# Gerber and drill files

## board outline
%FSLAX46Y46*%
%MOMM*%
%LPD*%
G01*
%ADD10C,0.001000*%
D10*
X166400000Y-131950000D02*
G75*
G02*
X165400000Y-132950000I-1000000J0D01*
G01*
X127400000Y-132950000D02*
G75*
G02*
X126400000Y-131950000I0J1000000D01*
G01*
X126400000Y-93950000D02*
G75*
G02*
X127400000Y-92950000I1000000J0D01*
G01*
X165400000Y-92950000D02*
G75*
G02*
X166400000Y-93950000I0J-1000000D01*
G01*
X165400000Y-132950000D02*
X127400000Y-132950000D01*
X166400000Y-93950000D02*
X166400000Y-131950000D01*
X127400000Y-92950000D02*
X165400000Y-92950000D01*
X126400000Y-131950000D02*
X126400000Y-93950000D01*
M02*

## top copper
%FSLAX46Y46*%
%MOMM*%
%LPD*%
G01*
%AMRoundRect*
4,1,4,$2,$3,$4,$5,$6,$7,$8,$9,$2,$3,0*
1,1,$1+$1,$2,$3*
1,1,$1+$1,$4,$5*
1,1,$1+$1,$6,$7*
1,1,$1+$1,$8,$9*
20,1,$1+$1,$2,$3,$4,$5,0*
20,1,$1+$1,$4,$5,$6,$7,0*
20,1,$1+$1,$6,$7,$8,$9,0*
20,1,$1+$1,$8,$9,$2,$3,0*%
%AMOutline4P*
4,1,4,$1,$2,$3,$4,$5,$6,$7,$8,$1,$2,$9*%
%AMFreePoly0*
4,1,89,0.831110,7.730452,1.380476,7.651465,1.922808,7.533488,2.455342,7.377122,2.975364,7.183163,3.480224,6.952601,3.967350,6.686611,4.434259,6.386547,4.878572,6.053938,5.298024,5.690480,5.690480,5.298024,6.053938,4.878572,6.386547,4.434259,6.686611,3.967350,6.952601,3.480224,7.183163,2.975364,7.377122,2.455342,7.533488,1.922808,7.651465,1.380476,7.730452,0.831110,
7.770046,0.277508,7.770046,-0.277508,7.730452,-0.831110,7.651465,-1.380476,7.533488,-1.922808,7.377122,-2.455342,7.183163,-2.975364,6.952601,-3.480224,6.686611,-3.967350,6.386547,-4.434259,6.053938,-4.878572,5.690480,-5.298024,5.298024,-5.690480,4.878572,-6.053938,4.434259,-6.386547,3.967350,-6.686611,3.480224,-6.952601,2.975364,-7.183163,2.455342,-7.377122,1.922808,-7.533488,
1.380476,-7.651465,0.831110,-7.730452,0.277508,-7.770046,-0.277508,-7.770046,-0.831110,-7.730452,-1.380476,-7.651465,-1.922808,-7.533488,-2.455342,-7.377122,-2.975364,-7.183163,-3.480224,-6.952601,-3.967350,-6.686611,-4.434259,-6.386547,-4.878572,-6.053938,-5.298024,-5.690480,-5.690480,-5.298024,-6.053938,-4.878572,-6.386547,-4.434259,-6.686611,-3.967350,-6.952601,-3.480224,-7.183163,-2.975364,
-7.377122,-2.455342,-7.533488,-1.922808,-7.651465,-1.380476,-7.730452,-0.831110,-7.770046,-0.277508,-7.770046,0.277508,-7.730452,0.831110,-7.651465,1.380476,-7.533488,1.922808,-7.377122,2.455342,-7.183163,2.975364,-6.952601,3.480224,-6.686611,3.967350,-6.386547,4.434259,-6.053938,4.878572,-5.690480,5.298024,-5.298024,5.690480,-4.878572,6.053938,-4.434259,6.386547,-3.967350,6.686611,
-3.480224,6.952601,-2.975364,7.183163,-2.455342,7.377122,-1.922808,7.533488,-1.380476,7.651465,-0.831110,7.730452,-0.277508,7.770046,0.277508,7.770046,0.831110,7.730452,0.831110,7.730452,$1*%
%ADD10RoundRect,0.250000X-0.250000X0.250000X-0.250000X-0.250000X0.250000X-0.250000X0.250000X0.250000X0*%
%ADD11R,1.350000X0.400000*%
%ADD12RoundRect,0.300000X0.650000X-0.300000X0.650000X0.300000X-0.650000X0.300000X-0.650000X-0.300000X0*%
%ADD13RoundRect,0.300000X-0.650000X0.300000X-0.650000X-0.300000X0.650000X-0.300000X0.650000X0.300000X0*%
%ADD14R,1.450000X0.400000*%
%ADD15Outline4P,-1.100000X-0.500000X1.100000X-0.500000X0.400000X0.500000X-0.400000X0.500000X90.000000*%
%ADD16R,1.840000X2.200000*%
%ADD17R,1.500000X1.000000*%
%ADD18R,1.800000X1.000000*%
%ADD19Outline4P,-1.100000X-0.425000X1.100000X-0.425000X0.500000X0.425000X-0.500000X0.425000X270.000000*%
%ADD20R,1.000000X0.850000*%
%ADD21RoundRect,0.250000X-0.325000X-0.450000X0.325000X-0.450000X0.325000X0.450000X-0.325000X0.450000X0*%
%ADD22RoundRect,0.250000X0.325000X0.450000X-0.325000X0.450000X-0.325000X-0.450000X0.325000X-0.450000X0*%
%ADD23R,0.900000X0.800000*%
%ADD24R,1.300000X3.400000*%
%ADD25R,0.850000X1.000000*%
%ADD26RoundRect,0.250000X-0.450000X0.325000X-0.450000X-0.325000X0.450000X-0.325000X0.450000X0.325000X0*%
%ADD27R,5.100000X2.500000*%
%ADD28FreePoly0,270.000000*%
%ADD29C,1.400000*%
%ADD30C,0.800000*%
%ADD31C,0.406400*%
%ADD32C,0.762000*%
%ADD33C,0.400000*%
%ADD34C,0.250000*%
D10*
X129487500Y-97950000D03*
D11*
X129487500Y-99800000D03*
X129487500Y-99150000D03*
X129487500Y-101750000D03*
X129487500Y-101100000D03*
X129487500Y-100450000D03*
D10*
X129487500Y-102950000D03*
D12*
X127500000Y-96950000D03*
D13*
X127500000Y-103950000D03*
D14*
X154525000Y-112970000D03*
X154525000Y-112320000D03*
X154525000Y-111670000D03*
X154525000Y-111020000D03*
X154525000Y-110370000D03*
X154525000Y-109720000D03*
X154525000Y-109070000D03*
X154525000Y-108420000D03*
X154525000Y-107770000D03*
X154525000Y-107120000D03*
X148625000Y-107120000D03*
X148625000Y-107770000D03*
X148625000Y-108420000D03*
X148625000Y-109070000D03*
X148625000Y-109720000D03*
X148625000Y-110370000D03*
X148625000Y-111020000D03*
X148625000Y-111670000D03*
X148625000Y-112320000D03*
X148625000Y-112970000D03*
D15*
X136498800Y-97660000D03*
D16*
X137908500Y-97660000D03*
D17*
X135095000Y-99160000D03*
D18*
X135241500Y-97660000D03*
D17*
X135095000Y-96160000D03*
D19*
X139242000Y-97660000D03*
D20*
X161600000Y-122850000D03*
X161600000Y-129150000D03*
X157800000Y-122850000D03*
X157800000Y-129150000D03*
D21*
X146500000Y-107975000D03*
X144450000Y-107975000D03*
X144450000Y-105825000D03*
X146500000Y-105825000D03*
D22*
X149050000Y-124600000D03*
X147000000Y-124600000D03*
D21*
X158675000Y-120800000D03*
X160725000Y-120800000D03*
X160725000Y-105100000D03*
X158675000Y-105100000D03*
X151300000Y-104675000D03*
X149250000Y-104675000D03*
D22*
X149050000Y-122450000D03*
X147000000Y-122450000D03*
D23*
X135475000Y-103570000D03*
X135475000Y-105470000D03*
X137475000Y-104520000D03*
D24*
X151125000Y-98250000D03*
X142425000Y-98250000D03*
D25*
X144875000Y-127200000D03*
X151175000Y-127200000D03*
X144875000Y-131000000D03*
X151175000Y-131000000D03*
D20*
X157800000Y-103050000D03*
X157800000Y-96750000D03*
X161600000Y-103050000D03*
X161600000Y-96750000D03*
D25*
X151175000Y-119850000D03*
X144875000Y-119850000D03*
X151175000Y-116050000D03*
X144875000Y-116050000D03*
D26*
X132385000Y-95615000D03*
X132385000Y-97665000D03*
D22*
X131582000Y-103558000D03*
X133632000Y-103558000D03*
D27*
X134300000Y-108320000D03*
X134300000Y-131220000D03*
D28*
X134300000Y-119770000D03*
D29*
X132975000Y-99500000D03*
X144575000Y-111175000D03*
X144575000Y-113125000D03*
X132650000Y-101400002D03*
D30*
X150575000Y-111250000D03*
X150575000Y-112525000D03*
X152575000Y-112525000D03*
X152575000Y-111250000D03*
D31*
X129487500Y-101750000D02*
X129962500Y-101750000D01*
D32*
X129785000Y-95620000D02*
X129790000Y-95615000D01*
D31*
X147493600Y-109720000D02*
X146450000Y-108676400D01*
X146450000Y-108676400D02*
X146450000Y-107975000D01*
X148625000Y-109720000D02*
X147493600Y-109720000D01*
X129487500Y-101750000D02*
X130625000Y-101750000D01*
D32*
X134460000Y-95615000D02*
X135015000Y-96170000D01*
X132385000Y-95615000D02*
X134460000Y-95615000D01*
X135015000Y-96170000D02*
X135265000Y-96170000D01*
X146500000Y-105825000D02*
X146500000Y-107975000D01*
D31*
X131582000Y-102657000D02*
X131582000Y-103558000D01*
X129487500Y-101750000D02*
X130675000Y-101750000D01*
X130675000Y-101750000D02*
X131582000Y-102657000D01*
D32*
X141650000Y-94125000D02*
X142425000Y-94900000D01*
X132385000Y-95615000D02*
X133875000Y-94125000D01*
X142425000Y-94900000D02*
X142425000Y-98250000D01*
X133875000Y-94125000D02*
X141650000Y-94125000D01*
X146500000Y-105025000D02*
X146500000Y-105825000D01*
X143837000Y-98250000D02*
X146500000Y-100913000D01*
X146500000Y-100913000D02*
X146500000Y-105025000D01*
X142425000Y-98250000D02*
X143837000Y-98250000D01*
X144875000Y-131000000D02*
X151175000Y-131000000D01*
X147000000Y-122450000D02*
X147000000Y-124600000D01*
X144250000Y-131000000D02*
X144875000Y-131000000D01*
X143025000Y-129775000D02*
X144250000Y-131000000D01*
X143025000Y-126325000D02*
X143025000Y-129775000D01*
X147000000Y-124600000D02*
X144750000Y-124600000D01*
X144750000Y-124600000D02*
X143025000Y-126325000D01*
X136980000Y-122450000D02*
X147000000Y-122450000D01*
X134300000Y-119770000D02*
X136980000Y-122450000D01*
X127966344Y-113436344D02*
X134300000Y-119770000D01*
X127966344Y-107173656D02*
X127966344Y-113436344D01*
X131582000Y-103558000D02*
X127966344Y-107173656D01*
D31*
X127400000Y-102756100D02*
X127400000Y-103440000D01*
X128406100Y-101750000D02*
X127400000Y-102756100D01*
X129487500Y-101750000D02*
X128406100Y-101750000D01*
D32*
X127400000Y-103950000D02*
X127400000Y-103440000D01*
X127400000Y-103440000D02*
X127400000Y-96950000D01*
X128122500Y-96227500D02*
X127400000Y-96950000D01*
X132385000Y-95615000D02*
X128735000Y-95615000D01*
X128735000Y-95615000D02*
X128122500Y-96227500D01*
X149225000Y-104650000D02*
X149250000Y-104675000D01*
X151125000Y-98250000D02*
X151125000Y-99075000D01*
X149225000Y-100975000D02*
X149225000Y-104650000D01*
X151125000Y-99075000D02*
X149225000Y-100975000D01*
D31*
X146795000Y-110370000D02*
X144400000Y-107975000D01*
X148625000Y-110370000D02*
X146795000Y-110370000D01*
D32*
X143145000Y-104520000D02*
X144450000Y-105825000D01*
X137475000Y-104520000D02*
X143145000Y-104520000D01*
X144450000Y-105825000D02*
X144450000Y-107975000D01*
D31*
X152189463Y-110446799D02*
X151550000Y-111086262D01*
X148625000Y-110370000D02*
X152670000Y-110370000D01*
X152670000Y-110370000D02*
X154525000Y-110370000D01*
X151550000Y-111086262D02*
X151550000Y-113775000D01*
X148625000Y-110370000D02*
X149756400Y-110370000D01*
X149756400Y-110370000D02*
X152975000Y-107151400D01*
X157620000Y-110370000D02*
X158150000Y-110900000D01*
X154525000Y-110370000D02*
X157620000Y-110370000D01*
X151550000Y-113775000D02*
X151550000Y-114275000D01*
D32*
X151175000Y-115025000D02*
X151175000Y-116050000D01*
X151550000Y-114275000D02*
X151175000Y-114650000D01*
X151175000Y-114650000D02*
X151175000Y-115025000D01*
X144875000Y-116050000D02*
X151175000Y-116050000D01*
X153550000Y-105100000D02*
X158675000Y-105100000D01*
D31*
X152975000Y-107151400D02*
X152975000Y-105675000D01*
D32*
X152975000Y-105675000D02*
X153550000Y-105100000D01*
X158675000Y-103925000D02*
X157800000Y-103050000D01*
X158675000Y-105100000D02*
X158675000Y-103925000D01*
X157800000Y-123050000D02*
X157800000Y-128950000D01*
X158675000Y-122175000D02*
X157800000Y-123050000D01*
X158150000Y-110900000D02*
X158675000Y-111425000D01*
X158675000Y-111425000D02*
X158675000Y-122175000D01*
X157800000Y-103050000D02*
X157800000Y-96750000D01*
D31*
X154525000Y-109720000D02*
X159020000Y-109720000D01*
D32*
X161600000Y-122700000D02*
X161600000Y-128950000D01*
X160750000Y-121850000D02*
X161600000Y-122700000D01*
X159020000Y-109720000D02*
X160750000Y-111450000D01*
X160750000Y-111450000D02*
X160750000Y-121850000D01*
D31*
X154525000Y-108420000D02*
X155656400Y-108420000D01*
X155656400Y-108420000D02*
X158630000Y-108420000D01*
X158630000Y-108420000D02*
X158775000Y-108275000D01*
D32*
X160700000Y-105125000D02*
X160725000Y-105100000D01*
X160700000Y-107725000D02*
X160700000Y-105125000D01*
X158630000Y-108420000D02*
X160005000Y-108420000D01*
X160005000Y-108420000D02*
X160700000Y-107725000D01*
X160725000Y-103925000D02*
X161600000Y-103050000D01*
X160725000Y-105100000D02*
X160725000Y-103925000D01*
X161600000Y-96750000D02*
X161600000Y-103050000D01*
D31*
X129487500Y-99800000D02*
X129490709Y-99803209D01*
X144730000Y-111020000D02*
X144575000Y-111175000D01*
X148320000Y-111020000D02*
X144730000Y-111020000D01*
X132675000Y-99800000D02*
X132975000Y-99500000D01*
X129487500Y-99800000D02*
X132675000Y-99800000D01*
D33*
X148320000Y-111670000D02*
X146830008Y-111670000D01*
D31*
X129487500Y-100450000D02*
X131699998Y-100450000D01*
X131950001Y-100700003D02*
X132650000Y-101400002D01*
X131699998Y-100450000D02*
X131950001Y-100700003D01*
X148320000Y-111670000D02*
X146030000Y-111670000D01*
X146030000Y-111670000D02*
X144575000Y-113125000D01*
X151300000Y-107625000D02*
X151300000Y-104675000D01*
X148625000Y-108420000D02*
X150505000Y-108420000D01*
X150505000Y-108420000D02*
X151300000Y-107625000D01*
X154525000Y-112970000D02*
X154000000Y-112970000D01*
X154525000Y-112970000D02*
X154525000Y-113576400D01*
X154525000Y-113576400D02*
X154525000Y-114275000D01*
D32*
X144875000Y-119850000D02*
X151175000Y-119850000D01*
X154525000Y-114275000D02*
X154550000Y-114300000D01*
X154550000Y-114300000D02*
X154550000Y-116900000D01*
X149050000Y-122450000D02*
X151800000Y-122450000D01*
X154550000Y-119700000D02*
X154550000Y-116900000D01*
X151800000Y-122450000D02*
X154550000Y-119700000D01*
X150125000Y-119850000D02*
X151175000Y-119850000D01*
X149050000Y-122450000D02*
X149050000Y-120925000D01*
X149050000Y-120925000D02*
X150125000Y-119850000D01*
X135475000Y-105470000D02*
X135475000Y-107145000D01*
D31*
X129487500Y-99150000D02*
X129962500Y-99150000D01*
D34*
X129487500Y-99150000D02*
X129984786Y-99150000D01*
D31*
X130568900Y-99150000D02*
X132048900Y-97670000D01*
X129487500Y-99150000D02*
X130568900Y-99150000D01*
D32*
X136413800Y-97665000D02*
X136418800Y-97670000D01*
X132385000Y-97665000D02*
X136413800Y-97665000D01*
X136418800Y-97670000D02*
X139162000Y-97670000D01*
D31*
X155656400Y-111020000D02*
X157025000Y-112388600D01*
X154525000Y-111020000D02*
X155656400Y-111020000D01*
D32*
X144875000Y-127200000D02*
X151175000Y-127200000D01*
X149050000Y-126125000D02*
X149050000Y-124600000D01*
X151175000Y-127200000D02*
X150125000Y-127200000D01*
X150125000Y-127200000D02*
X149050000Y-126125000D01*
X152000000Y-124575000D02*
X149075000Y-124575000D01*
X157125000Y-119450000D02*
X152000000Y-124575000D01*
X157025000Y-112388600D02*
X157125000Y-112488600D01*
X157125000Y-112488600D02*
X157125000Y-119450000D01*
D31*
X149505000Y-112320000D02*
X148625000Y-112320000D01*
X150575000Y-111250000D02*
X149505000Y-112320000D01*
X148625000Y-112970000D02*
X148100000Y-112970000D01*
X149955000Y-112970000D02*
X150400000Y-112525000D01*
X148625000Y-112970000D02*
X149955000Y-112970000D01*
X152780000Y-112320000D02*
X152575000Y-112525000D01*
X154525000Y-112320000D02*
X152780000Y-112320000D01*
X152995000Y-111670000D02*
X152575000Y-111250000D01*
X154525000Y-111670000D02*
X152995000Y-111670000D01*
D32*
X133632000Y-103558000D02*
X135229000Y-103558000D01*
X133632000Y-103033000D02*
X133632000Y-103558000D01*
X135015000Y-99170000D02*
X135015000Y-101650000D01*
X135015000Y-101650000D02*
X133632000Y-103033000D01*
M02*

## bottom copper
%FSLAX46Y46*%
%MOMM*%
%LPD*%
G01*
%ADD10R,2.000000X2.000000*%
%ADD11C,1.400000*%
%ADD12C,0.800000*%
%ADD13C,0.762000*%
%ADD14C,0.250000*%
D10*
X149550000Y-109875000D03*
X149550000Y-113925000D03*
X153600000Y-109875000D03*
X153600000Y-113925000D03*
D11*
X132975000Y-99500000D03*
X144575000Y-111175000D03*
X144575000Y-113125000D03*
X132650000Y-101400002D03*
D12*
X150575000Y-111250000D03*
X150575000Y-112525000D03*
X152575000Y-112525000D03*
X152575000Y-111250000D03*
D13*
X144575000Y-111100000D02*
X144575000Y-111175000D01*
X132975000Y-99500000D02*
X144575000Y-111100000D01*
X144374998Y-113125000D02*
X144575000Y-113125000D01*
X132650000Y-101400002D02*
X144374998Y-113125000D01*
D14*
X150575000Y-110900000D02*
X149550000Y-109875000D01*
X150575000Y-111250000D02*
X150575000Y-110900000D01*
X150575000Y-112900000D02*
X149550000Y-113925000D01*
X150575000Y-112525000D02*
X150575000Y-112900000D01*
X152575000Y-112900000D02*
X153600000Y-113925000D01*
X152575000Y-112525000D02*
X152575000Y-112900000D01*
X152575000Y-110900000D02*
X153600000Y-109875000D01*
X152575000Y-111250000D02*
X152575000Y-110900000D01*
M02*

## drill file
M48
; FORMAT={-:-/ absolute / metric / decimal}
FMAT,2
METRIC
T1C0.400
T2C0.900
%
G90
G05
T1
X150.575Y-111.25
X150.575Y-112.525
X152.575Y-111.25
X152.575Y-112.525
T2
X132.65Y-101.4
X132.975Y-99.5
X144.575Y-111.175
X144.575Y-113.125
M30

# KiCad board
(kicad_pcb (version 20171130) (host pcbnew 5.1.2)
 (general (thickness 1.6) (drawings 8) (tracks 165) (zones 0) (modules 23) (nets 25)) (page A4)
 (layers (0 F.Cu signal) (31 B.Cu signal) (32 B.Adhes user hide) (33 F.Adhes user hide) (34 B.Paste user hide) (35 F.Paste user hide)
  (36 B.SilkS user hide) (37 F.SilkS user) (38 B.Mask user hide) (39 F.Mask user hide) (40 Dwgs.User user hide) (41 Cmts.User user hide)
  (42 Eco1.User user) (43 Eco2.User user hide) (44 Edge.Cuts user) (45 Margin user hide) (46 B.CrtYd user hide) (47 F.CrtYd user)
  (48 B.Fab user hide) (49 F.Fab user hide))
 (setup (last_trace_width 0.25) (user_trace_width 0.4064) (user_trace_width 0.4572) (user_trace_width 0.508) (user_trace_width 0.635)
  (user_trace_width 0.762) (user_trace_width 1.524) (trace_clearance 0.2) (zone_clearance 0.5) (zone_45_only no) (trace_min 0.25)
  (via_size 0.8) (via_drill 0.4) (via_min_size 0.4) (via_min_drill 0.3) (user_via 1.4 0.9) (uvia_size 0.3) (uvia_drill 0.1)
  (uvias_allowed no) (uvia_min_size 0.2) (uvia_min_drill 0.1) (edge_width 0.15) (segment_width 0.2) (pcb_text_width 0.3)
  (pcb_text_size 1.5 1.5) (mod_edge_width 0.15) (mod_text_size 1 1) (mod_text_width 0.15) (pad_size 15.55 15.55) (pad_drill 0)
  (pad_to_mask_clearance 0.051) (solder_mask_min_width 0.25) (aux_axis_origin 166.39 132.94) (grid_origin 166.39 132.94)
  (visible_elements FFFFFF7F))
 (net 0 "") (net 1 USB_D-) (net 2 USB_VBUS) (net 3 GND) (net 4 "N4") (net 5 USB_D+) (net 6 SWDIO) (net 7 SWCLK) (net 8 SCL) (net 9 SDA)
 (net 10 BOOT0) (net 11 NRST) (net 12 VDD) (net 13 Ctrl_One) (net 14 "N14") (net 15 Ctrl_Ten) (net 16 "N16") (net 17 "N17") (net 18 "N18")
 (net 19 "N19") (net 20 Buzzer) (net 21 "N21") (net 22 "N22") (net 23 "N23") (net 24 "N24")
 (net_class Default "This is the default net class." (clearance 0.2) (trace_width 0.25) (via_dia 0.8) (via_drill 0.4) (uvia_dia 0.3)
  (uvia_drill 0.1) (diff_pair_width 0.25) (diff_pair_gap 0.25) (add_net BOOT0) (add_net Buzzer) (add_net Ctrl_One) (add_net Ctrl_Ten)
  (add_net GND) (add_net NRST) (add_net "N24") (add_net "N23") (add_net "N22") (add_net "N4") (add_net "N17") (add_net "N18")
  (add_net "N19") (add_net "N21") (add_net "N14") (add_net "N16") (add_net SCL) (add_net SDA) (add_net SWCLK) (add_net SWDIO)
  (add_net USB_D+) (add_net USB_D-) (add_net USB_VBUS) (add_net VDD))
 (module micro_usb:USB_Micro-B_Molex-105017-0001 (layer F.Cu) (at 128.025 100.45 270)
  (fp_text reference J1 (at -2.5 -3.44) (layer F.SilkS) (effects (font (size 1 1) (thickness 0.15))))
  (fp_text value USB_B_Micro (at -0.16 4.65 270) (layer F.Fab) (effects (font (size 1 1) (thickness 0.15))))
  (pad "" smd roundrect (at -2.5 -1.4625 270) (size 1 1) (layers F.Cu F.Paste F.Mask) (roundrect_rratio 0.25))
  (pad 2 smd rect (at -0.65 -1.4625 270) (size 0.4 1.35) (layers F.Cu F.Paste F.Mask) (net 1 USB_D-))
  (pad 1 smd rect (at -1.3 -1.4625 270) (size 0.4 1.35) (layers F.Cu F.Paste F.Mask) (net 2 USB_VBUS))
  (pad 5 smd rect (at 1.3 -1.4625 270) (size 0.4 1.35) (layers F.Cu F.Paste F.Mask) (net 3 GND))
  (pad 4 smd rect (at 0.65 -1.4625 270) (size 0.4 1.35) (layers F.Cu F.Paste F.Mask) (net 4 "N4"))
  (pad 3 smd rect (at 0 -1.4625 270) (size 0.4 1.35) (layers F.Cu F.Paste F.Mask) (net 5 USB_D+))
  (pad "" smd roundrect (at 2.5 -1.4625 270) (size 1 1) (layers F.Cu F.Paste F.Mask) (roundrect_rratio 0.25))
  (pad 6 smd roundrect (at -3.5 0.525 90) (size 1.2 1.9) (layers F.Cu F.Paste F.Mask) (roundrect_rratio 0.25) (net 3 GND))
  (pad 6 smd roundrect (at 3.5 0.525 270) (size 1.2 1.9) (layers F.Cu F.Paste F.Mask) (roundrect_rratio 0.25) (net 3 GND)))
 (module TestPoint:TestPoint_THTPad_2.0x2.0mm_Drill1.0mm (layer B.Cu) (at 149.55 109.875 180)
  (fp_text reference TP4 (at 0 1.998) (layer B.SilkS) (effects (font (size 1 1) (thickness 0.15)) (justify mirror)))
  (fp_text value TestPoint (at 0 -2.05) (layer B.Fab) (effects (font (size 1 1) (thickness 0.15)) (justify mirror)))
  (pad 1 smd rect (at 0 0 180) (size 2 2) (layers B.Cu B.Paste B.Mask) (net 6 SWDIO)))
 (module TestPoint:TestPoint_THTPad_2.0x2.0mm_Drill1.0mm (layer B.Cu) (at 149.55 113.925 180)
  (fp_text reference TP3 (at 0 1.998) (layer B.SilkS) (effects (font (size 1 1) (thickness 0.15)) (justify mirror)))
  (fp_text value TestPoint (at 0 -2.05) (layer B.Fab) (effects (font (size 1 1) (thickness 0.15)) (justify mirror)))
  (pad 1 smd rect (at 0 0 180) (size 2 2) (layers B.Cu B.Paste B.Mask) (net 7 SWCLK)))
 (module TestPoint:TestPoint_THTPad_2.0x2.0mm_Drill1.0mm (layer B.Cu) (at 153.6 109.875 180)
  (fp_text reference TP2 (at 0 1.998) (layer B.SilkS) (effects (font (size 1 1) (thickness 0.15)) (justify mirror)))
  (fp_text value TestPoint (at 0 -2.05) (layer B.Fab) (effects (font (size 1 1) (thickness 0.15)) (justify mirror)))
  (pad 1 smd rect (at 0 0 180) (size 2 2) (layers B.Cu B.Paste B.Mask) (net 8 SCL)))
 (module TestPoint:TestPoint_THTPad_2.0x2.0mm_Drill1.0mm (layer B.Cu) (at 153.6 113.925 180)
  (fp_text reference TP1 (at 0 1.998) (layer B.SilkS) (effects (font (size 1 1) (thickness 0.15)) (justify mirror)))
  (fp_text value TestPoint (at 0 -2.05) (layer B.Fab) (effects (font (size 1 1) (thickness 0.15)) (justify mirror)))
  (pad 1 smd rect (at 0 0 180) (size 2 2) (layers B.Cu B.Paste B.Mask) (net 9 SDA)))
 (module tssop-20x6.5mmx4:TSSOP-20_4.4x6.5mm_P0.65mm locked (layer F.Cu) (at 151.575 110.045 180)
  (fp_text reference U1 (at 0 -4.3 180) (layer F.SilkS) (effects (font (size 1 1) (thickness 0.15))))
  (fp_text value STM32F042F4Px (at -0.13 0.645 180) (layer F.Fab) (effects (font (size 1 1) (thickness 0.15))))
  (pad 1 smd rect (at -2.95 -2.925 180) (size 1.45 0.4) (layers F.Cu F.Paste F.Mask) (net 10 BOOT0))
  (pad 2 smd rect (at -2.95 -2.275 180) (size 1.45 0.4) (layers F.Cu F.Paste F.Mask) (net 9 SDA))
  (pad 3 smd rect (at -2.95 -1.625 180) (size 1.45 0.4) (layers F.Cu F.Paste F.Mask) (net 8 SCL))
  (pad 4 smd rect (at -2.95 -0.975 180) (size 1.45 0.4) (layers F.Cu F.Paste F.Mask) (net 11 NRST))
  (pad 5 smd rect (at -2.95 -0.325 180) (size 1.45 0.4) (layers F.Cu F.Paste F.Mask) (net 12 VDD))
  (pad 6 smd rect (at -2.95 0.325 180) (size 1.45 0.4) (layers F.Cu F.Paste F.Mask) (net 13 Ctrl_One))
  (pad 7 smd rect (at -2.95 0.975 180) (size 1.45 0.4) (layers F.Cu F.Paste F.Mask) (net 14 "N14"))
  (pad 8 smd rect (at -2.95 1.625 180) (size 1.45 0.4) (layers F.Cu F.Paste F.Mask) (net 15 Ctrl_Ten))
  (pad 9 smd rect (at -2.95 2.275 180) (size 1.45 0.4) (layers F.Cu F.Paste F.Mask) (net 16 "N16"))
  (pad 10 smd rect (at -2.95 2.925 180) (size 1.45 0.4) (layers F.Cu F.Paste F.Mask) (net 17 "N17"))
  (pad 11 smd rect (at 2.95 2.925 180) (size 1.45 0.4) (layers F.Cu F.Paste F.Mask) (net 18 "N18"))
  (pad 12 smd rect (at 2.95 2.275 180) (size 1.45 0.4) (layers F.Cu F.Paste F.Mask) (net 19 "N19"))
  (pad 13 smd rect (at 2.95 1.625 180) (size 1.45 0.4) (layers F.Cu F.Paste F.Mask) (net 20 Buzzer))
  (pad 14 smd rect (at 2.95 0.975 180) (size 1.45 0.4) (layers F.Cu F.Paste F.Mask) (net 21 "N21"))
  (pad 15 smd rect (at 2.95 0.325 180) (size 1.45 0.4) (layers F.Cu F.Paste F.Mask) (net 3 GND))
  (pad 16 smd rect (at 2.95 -0.325 180) (size 1.45 0.4) (layers F.Cu F.Paste F.Mask) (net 12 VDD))
  (pad 17 smd rect (at 2.95 -0.975 180) (size 1.45 0.4) (layers F.Cu F.Paste F.Mask) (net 1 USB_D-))
  (pad 18 smd rect (at 2.95 -1.625 180) (size 1.45 0.4) (layers F.Cu F.Paste F.Mask) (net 5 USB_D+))
  (pad 19 smd rect (at 2.95 -2.275 180) (size 1.45 0.4) (layers F.Cu F.Paste F.Mask) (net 6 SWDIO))
  (pad 20 smd rect (at 2.95 -2.925 180) (size 1.45 0.4) (layers F.Cu F.Paste F.Mask) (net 7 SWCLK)))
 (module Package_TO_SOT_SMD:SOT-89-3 (layer F.Cu) (at 136.575 97.66)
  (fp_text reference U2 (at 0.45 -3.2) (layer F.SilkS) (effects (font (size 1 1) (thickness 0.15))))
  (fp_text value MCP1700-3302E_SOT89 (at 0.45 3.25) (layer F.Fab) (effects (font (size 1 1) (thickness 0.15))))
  (pad 2 smd trapezoid (at -0.0762 0 90) (size 1.5 1) (rect_delta 0 0.7) (layers F.Cu F.Paste F.Mask) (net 2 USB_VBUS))
  (pad 2 smd rect (at 1.3335 0 270) (size 2.2 1.84) (layers F.Cu F.Paste F.Mask) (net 2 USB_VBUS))
  (pad 3 smd rect (at -1.48 1.5 270) (size 1 1.5) (layers F.Cu F.Paste F.Mask) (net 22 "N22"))
  (pad 2 smd rect (at -1.3335 0 270) (size 1 1.8) (layers F.Cu F.Paste F.Mask) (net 2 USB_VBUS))
  (pad 1 smd rect (at -1.48 -1.5 270) (size 1 1.5) (layers F.Cu F.Paste F.Mask) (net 3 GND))
  (pad 2 smd trapezoid (at 2.667 0 270) (size 1.6 0.85) (rect_delta 0 0.6) (layers F.Cu F.Paste F.Mask) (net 2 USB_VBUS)))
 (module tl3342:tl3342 (layer F.Cu) (at 159.7 126 270)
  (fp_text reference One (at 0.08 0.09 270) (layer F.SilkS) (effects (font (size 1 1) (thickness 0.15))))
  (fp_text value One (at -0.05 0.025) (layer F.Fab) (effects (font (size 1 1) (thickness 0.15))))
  (pad 1 smd rect (at -3.15 -1.9 270) (size 0.85 1) (layers F.Cu F.Paste F.Mask) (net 13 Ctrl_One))
  (pad 1 smd rect (at 3.15 -1.9 270) (size 0.85 1) (layers F.Cu F.Paste F.Mask) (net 13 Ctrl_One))
  (pad 2 smd rect (at -3.15 1.9 270) (size 0.85 1) (layers F.Cu F.Paste F.Mask) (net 12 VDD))
  (pad 2 smd rect (at 3.15 1.9 270) (size 0.85 1) (layers F.Cu F.Paste F.Mask) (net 12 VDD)))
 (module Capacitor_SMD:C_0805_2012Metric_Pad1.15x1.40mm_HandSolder (layer F.Cu) (at 145.475 107.975)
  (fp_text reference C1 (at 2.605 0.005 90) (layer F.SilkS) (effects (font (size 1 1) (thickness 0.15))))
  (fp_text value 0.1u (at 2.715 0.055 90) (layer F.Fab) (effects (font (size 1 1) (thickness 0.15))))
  (pad 2 smd roundrect (at 1.025 0) (size 1.15 1.4) (layers F.Cu F.Paste F.Mask) (roundrect_rratio 0.217391) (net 3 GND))
  (pad 1 smd roundrect (at -1.025 0) (size 1.15 1.4) (layers F.Cu F.Paste F.Mask) (roundrect_rratio 0.217391) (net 12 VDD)))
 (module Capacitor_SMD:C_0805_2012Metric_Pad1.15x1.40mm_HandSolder (layer F.Cu) (at 145.475 105.825)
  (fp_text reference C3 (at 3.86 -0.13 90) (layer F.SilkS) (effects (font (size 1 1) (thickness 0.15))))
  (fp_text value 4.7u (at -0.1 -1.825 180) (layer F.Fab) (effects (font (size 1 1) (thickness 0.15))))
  (pad 1 smd roundrect (at -1.025 0) (size 1.15 1.4) (layers F.Cu F.Paste F.Mask) (roundrect_rratio 0.217391) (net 12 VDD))
  (pad 2 smd roundrect (at 1.025 0) (size 1.15 1.4) (layers F.Cu F.Paste F.Mask) (roundrect_rratio 0.217391) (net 3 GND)))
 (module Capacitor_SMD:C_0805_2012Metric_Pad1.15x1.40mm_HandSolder (layer F.Cu) (at 148.025 124.6 180)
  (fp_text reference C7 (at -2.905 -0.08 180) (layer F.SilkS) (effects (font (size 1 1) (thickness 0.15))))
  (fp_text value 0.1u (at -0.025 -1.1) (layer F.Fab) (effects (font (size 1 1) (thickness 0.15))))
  (pad 1 smd roundrect (at -1.025 0 180) (size 1.15 1.4) (layers F.Cu F.Paste F.Mask) (roundrect_rratio 0.217391) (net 11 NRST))
  (pad 2 smd roundrect (at 1.025 0 180) (size 1.15 1.4) (layers F.Cu F.Paste F.Mask) (roundrect_rratio 0.217391) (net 3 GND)))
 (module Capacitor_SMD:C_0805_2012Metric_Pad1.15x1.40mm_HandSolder (layer F.Cu) (at 159.7 120.8)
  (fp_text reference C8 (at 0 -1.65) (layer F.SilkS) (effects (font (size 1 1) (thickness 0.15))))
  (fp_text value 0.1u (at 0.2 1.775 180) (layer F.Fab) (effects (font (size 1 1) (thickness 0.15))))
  (pad 1 smd roundrect (at -1.025 0) (size 1.15 1.4) (layers F.Cu F.Paste F.Mask) (roundrect_rratio 0.217391) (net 12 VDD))
  (pad 2 smd roundrect (at 1.025 0) (size 1.15 1.4) (layers F.Cu F.Paste F.Mask) (roundrect_rratio 0.217391) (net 13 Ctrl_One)))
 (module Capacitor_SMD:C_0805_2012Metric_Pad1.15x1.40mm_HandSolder (layer F.Cu) (at 159.7 105.1)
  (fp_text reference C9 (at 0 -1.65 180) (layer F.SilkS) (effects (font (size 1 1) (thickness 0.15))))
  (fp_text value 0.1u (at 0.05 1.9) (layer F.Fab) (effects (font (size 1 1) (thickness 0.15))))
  (pad 2 smd roundrect (at 1.025 0) (size 1.15 1.4) (layers F.Cu F.Paste F.Mask) (roundrect_rratio 0.217391) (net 15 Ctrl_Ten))
  (pad 1 smd roundrect (at -1.025 0) (size 1.15 1.4) (layers F.Cu F.Paste F.Mask) (roundrect_rratio 0.217391) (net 12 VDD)))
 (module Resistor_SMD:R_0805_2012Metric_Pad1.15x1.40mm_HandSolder (layer F.Cu) (at 150.275 104.675)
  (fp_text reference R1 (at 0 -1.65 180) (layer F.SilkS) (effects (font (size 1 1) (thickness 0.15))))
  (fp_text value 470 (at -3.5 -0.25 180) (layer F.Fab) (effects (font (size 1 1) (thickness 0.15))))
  (pad 2 smd roundrect (at 1.025 0) (size 1.15 1.4) (layers F.Cu F.Paste F.Mask) (roundrect_rratio 0.217391) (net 20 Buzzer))
  (pad 1 smd roundrect (at -1.025 0) (size 1.15 1.4) (layers F.Cu F.Paste F.Mask) (roundrect_rratio 0.217391) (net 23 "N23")))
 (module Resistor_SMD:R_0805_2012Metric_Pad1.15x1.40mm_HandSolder (layer F.Cu) (at 148.025 122.45 180)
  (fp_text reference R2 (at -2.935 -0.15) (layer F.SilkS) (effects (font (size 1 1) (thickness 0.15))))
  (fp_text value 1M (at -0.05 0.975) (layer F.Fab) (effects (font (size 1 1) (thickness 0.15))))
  (pad 1 smd roundrect (at -1.025 0 180) (size 1.15 1.4) (layers F.Cu F.Paste F.Mask) (roundrect_rratio 0.217391) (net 10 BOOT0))
  (pad 2 smd roundrect (at 1.025 0 180) (size 1.15 1.4) (layers F.Cu F.Paste F.Mask) (roundrect_rratio 0.217391) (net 3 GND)))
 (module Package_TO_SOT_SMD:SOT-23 (layer F.Cu) (at 136.475 104.52)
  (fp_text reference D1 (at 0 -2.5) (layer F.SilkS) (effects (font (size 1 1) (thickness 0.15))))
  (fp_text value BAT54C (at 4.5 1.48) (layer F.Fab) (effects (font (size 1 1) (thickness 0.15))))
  (pad 1 smd rect (at -1 -0.95) (size 0.9 0.8) (layers F.Cu F.Paste F.Mask) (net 22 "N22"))
  (pad 2 smd rect (at -1 0.95) (size 0.9 0.8) (layers F.Cu F.Paste F.Mask) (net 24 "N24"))
  (pad 3 smd rect (at 1 0) (size 0.9 0.8) (layers F.Cu F.Paste F.Mask) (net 12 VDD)))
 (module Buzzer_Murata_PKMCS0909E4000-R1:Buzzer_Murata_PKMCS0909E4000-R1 (layer F.Cu) (at 146.775 98.25 180)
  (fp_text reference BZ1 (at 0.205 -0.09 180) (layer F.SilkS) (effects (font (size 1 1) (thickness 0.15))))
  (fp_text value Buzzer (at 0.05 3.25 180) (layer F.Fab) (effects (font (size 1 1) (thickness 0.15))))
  (pad 1 smd rect (at -4.35 0 180) (size 1.3 3.4) (layers F.Cu F.Paste F.Mask) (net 23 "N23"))
  (pad 2 smd rect (at 4.35 0 180) (size 1.3 3.4) (layers F.Cu F.Paste F.Mask) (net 3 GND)))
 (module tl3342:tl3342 (layer F.Cu) (at 148.025 129.1)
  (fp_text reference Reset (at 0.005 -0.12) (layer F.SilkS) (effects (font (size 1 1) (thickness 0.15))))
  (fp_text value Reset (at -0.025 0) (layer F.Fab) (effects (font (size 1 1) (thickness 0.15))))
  (pad 1 smd rect (at -3.15 -1.9) (size 0.85 1) (layers F.Cu F.Paste F.Mask) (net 11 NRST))
  (pad 1 smd rect (at 3.15 -1.9) (size 0.85 1) (layers F.Cu F.Paste F.Mask) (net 11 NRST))
  (pad 2 smd rect (at -3.15 1.9) (size 0.85 1) (layers F.Cu F.Paste F.Mask) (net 3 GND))
  (pad 2 smd rect (at 3.15 1.9) (size 0.85 1) (layers F.Cu F.Paste F.Mask) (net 3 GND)))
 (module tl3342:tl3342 (layer F.Cu) (at 159.7 99.9 270)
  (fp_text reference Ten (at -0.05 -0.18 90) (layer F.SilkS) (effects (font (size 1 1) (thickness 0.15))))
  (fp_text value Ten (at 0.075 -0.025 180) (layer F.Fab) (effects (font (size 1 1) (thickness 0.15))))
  (pad 2 smd rect (at 3.15 1.9 270) (size 0.85 1) (layers F.Cu F.Paste F.Mask) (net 12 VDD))
  (pad 2 smd rect (at -3.15 1.9 270) (size 0.85 1) (layers F.Cu F.Paste F.Mask) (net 12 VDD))
  (pad 1 smd rect (at 3.15 -1.9 270) (size 0.85 1) (layers F.Cu F.Paste F.Mask) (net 15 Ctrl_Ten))
  (pad 1 smd rect (at -3.15 -1.9 270) (size 0.85 1) (layers F.Cu F.Paste F.Mask) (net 15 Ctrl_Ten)))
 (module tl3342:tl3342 (layer F.Cu) (at 148.025 117.95 180)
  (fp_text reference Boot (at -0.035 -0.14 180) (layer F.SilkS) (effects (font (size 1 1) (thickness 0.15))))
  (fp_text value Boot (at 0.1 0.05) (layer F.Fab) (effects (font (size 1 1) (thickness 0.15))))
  (pad 1 smd rect (at -3.15 -1.9 180) (size 0.85 1) (layers F.Cu F.Paste F.Mask) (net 10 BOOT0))
  (pad 1 smd rect (at 3.15 -1.9 180) (size 0.85 1) (layers F.Cu F.Paste F.Mask) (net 10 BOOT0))
  (pad 2 smd rect (at -3.15 1.9 180) (size 0.85 1) (layers F.Cu F.Paste F.Mask) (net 12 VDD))
  (pad 2 smd rect (at 3.15 1.9 180) (size 0.85 1) (layers F.Cu F.Paste F.Mask) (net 12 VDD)))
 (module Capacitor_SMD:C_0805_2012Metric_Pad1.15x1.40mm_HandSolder (layer F.Cu) (at 132.385 96.64 270)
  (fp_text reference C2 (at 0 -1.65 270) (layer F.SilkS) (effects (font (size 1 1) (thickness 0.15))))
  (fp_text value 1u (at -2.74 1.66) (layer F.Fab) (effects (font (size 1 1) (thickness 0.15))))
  (pad 1 smd roundrect (at -1.025 0 270) (size 1.15 1.4) (layers F.Cu F.Paste F.Mask) (roundrect_rratio 0.217391) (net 3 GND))
  (pad 2 smd roundrect (at 1.025 0 270) (size 1.15 1.4) (layers F.Cu F.Paste F.Mask) (roundrect_rratio 0.217391) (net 2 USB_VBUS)))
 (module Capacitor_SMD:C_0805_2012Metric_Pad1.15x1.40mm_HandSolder (layer F.Cu) (at 132.607 103.558 180)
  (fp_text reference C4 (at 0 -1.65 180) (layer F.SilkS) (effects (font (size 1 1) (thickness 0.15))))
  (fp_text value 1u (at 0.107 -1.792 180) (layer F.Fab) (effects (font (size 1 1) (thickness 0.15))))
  (pad 2 smd roundrect (at 1.025 0 180) (size 1.15 1.4) (layers F.Cu F.Paste F.Mask) (roundrect_rratio 0.217391) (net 3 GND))
  (pad 1 smd roundrect (at -1.025 0 180) (size 1.15 1.4) (layers F.Cu F.Paste F.Mask) (roundrect_rratio 0.217391) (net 22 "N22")))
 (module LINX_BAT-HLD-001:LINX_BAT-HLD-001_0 (layer F.Cu) (at 134.3 119.77 270)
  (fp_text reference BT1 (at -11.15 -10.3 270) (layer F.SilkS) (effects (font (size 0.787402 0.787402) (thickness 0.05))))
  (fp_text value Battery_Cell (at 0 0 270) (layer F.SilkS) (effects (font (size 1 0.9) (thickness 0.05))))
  (pad 1 smd rect (at -11.45 0 270) (size 2.5 5.1) (layers F.Cu F.Paste F.Mask) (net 24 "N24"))
  (pad 1 smd rect (at 11.45 0 270) (size 2.5 5.1) (layers F.Cu F.Paste F.Mask))
  (pad 2 smd custom (at 0 0 270) (size 15.55 15.55) (layers F.Cu F.Paste F.Mask) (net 3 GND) (zone_connect 0)
   (options (clearance outline) (anchor circle)) (primitives)))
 (gr_arc (start 165.4 131.95) (end 165.4 132.95) (angle -90) (layer Edge.Cuts) (width 0.001))
 (gr_arc (start 127.4 131.95) (end 126.4 131.95) (angle -90) (layer Edge.Cuts) (width 0.001))
 (gr_arc (start 127.4 93.95) (end 127.4 92.95) (angle -90) (layer Edge.Cuts) (width 0.001))
 (gr_arc (start 165.4 93.95) (end 165.4 92.95) (angle 90) (layer Edge.Cuts) (width 0.001))
 (gr_line (start 165.4 132.95) (end 127.4 132.95) (layer Edge.Cuts) (width 0.001))
 (gr_line (start 166.4 93.95) (end 166.4 131.95) (layer Edge.Cuts) (width 0.001))
 (gr_line (start 127.4 92.95) (end 165.4 92.95) (layer Edge.Cuts) (width 0.001))
 (gr_line (start 126.4 131.95) (end 126.4 93.95) (layer Edge.Cuts) (width 0.001))
 (segment (start 129.4875 101.75) (end 129.9625 101.75) (width 0.4064) (layer F.Cu) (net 3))
 (segment (start 129.785 95.62) (end 129.79 95.615) (width 0.762) (layer F.Cu) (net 3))
 (segment (start 147.4936 109.72) (end 146.45 108.6764) (width 0.4064) (layer F.Cu) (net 3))
 (segment (start 146.45 108.6764) (end 146.45 107.975) (width 0.4064) (layer F.Cu) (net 3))
 (segment (start 148.625 109.72) (end 147.4936 109.72) (width 0.4064) (layer F.Cu) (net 3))
 (segment (start 129.4875 101.75) (end 130.625 101.75) (width 0.4064) (layer F.Cu) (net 3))
 (segment (start 134.46 95.615) (end 135.015 96.17) (width 0.762) (layer F.Cu) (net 3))
 (segment (start 132.385 95.615) (end 134.46 95.615) (width 0.762) (layer F.Cu) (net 3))
 (segment (start 135.015 96.17) (end 135.265 96.17) (width 0.762) (layer F.Cu) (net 3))
 (segment (start 146.5 105.825) (end 146.5 107.975) (width 0.762) (layer F.Cu) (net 3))
 (segment (start 131.582 102.657) (end 131.582 103.558) (width 0.4064) (layer F.Cu) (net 3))
 (segment (start 129.4875 101.75) (end 130.675 101.75) (width 0.4064) (layer F.Cu) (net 3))
 (segment (start 130.675 101.75) (end 131.582 102.657) (width 0.4064) (layer F.Cu) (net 3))
 (segment (start 141.65 94.125) (end 142.425 94.9) (width 0.762) (layer F.Cu) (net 3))
 (segment (start 132.385 95.615) (end 133.875 94.125) (width 0.762) (layer F.Cu) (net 3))
 (segment (start 142.425 94.9) (end 142.425 98.25) (width 0.762) (layer F.Cu) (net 3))
 (segment (start 133.875 94.125) (end 141.65 94.125) (width 0.762) (layer F.Cu) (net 3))
 (segment (start 146.5 105.025) (end 146.5 105.825) (width 0.762) (layer F.Cu) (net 3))
 (segment (start 143.837 98.25) (end 146.5 100.913) (width 0.762) (layer F.Cu) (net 3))
 (segment (start 146.5 100.913) (end 146.5 105.025) (width 0.762) (layer F.Cu) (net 3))
 (segment (start 142.425 98.25) (end 143.837 98.25) (width 0.762) (layer F.Cu) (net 3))
 (segment (start 144.875 131) (end 151.175 131) (width 0.762) (layer F.Cu) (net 3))
 (segment (start 147 122.45) (end 147 124.6) (width 0.762) (layer F.Cu) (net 3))
 (segment (start 144.25 131) (end 144.875 131) (width 0.762) (layer F.Cu) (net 3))
 (segment (start 143.025 129.775) (end 144.25 131) (width 0.762) (layer F.Cu) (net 3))
 (segment (start 143.025 126.325) (end 143.025 129.775) (width 0.762) (layer F.Cu) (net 3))
 (segment (start 147 124.6) (end 144.75 124.6) (width 0.762) (layer F.Cu) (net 3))
 (segment (start 144.75 124.6) (end 143.025 126.325) (width 0.762) (layer F.Cu) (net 3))
 (segment (start 136.98 122.45) (end 147 122.45) (width 0.762) (layer F.Cu) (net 3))
 (segment (start 134.3 119.77) (end 136.98 122.45) (width 0.762) (layer F.Cu) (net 3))
 (segment (start 127.966344 113.436344) (end 134.3 119.77) (width 0.762) (layer F.Cu) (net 3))
 (segment (start 127.966344 107.173656) (end 127.966344 113.436344) (width 0.762) (layer F.Cu) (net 3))
 (segment (start 131.582 103.558) (end 127.966344 107.173656) (width 0.762) (layer F.Cu) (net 3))
 (segment (start 127.4 102.7561) (end 127.4 103.44) (width 0.4064) (layer F.Cu) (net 3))
 (segment (start 128.4061 101.75) (end 127.4 102.7561) (width 0.4064) (layer F.Cu) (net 3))
 (segment (start 129.4875 101.75) (end 128.4061 101.75) (width 0.4064) (layer F.Cu) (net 3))
 (segment (start 127.4 103.95) (end 127.4 103.44) (width 0.762) (layer F.Cu) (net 3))
 (segment (start 127.4 103.44) (end 127.4 96.95) (width 0.762) (layer F.Cu) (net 3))
 (segment (start 128.1225 96.2275) (end 127.4 96.95) (width 0.762) (layer F.Cu) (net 3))
 (segment (start 132.385 95.615) (end 128.735 95.615) (width 0.762) (layer F.Cu) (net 3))
 (segment (start 128.735 95.615) (end 128.1225 96.2275) (width 0.762) (layer F.Cu) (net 3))
 (segment (start 149.225 104.65) (end 149.25 104.675) (width 0.762) (layer F.Cu) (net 23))
 (segment (start 151.125 98.25) (end 151.125 99.075) (width 0.762) (layer F.Cu) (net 23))
 (segment (start 149.225 100.975) (end 149.225 104.65) (width 0.762) (layer F.Cu) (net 23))
 (segment (start 151.125 99.075) (end 149.225 100.975) (width 0.762) (layer F.Cu) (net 23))
 (segment (start 146.795 110.37) (end 144.4 107.975) (width 0.4064) (layer F.Cu) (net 12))
 (segment (start 148.625 110.37) (end 146.795 110.37) (width 0.4064) (layer F.Cu) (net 12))
 (segment (start 143.145 104.52) (end 144.45 105.825) (width 0.762) (layer F.Cu) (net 12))
 (segment (start 137.475 104.52) (end 143.145 104.52) (width 0.762) (layer F.Cu) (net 12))
 (segment (start 144.45 105.825) (end 144.45 107.975) (width 0.762) (layer F.Cu) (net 12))
 (segment (start 152.189463 110.446799) (end 151.55 111.086262) (width 0.4064) (layer F.Cu) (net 12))
 (segment (start 148.625 110.37) (end 152.67 110.37) (width 0.4064) (layer F.Cu) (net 12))
 (segment (start 152.67 110.37) (end 154.525 110.37) (width 0.4064) (layer F.Cu) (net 12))
 (segment (start 151.55 111.086262) (end 151.55 113.775) (width 0.4064) (layer F.Cu) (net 12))
 (segment (start 148.625 110.37) (end 149.7564 110.37) (width 0.4064) (layer F.Cu) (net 12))
 (segment (start 149.7564 110.37) (end 152.975 107.1514) (width 0.4064) (layer F.Cu) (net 12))
 (segment (start 157.62 110.37) (end 158.15 110.9) (width 0.4064) (layer F.Cu) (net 12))
 (segment (start 154.525 110.37) (end 157.62 110.37) (width 0.4064) (layer F.Cu) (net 12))
 (segment (start 151.55 113.775) (end 151.55 114.275) (width 0.4064) (layer F.Cu) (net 12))
 (segment (start 151.175 115.025) (end 151.175 116.05) (width 0.762) (layer F.Cu) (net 12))
 (segment (start 151.55 114.275) (end 151.175 114.65) (width 0.762) (layer F.Cu) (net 12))
 (segment (start 151.175 114.65) (end 151.175 115.025) (width 0.762) (layer F.Cu) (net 12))
 (segment (start 144.875 116.05) (end 151.175 116.05) (width 0.762) (layer F.Cu) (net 12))
 (segment (start 153.55 105.1) (end 158.675 105.1) (width 0.762) (layer F.Cu) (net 12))
 (segment (start 152.975 107.1514) (end 152.975 105.675) (width 0.4064) (layer F.Cu) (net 12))
 (segment (start 152.975 105.675) (end 153.55 105.1) (width 0.762) (layer F.Cu) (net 12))
 (segment (start 158.675 103.925) (end 157.8 103.05) (width 0.762) (layer F.Cu) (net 12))
 (segment (start 158.675 105.1) (end 158.675 103.925) (width 0.762) (layer F.Cu) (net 12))
 (segment (start 157.8 123.05) (end 157.8 128.95) (width 0.762) (layer F.Cu) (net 12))
 (segment (start 158.675 122.175) (end 157.8 123.05) (width 0.762) (layer F.Cu) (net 12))
 (segment (start 158.15 110.9) (end 158.675 111.425) (width 0.762) (layer F.Cu) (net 12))
 (segment (start 158.675 111.425) (end 158.675 122.175) (width 0.762) (layer F.Cu) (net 12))
 (segment (start 157.8 103.05) (end 157.8 96.75) (width 0.762) (layer F.Cu) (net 12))
 (segment (start 154.525 109.72) (end 159.02 109.72) (width 0.4064) (layer F.Cu) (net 13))
 (segment (start 161.6 122.7) (end 161.6 128.95) (width 0.762) (layer F.Cu) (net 13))
 (segment (start 160.75 121.85) (end 161.6 122.7) (width 0.762) (layer F.Cu) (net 13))
 (segment (start 159.02 109.72) (end 160.75 111.45) (width 0.762) (layer F.Cu) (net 13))
 (segment (start 160.75 111.45) (end 160.75 121.85) (width 0.762) (layer F.Cu) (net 13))
 (segment (start 154.525 108.42) (end 155.6564 108.42) (width 0.4064) (layer F.Cu) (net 15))
 (segment (start 155.6564 108.42) (end 158.63 108.42) (width 0.4064) (layer F.Cu) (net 15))
 (segment (start 158.63 108.42) (end 158.775 108.275) (width 0.4064) (layer F.Cu) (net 15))
 (segment (start 160.7 105.125) (end 160.725 105.1) (width 0.762) (layer F.Cu) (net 15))
 (segment (start 160.7 107.725) (end 160.7 105.125) (width 0.762) (layer F.Cu) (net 15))
 (segment (start 158.63 108.42) (end 160.005 108.42) (width 0.762) (layer F.Cu) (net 15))
 (segment (start 160.005 108.42) (end 160.7 107.725) (width 0.762) (layer F.Cu) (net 15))
 (segment (start 160.725 103.925) (end 161.6 103.05) (width 0.762) (layer F.Cu) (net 15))
 (segment (start 160.725 105.1) (end 160.725 103.925) (width 0.762) (layer F.Cu) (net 15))
 (segment (start 161.6 96.75) (end 161.6 103.05) (width 0.762) (layer F.Cu) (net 15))
 (segment (start 129.4875 99.8) (end 129.490709 99.803209) (width 0.4064) (layer F.Cu) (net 1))
 (via (at 132.975 99.5) (size 1.4) (drill 0.9) (layers F.Cu B.Cu) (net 1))
 (via (at 144.575 111.175) (size 1.4) (drill 0.9) (layers F.Cu B.Cu) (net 1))
 (segment (start 144.73 111.02) (end 144.575 111.175) (width 0.4064) (layer F.Cu) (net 1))
 (segment (start 148.32 111.02) (end 144.73 111.02) (width 0.4064) (layer F.Cu) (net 1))
 (segment (start 132.675 99.8) (end 132.975 99.5) (width 0.4064) (layer F.Cu) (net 1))
 (segment (start 129.4875 99.8) (end 132.675 99.8) (width 0.4064) (layer F.Cu) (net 1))
 (segment (start 144.575 111.1) (end 144.575 111.175) (width 0.762) (layer B.Cu) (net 1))
 (segment (start 132.975 99.5) (end 144.575 111.1) (width 0.762) (layer B.Cu) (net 1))
 (segment (start 148.32 111.67) (end 146.830008 111.67) (width 0.4) (layer F.Cu) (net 5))
 (via (at 144.575 113.125) (size 1.4) (drill 0.9) (layers F.Cu B.Cu) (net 5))
 (via (at 132.65 101.400002) (size 1.4) (drill 0.9) (layers F.Cu B.Cu) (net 5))
 (segment (start 129.4875 100.45) (end 131.699998 100.45) (width 0.4064) (layer F.Cu) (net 5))
 (segment (start 131.950001 100.700003) (end 132.65 101.400002) (width 0.4064) (layer F.Cu) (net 5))
 (segment (start 131.699998 100.45) (end 131.950001 100.700003) (width 0.4064) (layer F.Cu) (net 5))
 (segment (start 144.374998 113.125) (end 144.575 113.125) (width 0.762) (layer B.Cu) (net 5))
 (segment (start 132.65 101.400002) (end 144.374998 113.125) (width 0.762) (layer B.Cu) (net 5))
 (segment (start 148.32 111.67) (end 146.03 111.67) (width 0.4064) (layer F.Cu) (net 5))
 (segment (start 146.03 111.67) (end 144.575 113.125) (width 0.4064) (layer F.Cu) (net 5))
 (segment (start 151.3 107.625) (end 151.3 104.675) (width 0.4064) (layer F.Cu) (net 20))
 (segment (start 148.625 108.42) (end 150.505 108.42) (width 0.4064) (layer F.Cu) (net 20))
 (segment (start 150.505 108.42) (end 151.3 107.625) (width 0.4064) (layer F.Cu) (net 20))
 (segment (start 154.525 112.97) (end 154 112.97) (width 0.4064) (layer F.Cu) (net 10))
 (segment (start 154.525 112.97) (end 154.525 113.5764) (width 0.4064) (layer F.Cu) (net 10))
 (segment (start 154.525 113.5764) (end 154.525 114.275) (width 0.4064) (layer F.Cu) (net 10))
 (segment (start 144.875 119.85) (end 151.175 119.85) (width 0.762) (layer F.Cu) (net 10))
 (segment (start 154.525 114.275) (end 154.55 114.3) (width 0.762) (layer F.Cu) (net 10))
 (segment (start 154.55 114.3) (end 154.55 116.9) (width 0.762) (layer F.Cu) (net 10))
 (segment (start 149.05 122.45) (end 151.8 122.45) (width 0.762) (layer F.Cu) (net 10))
 (segment (start 154.55 119.7) (end 154.55 116.9) (width 0.762) (layer F.Cu) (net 10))
 (segment (start 151.8 122.45) (end 154.55 119.7) (width 0.762) (layer F.Cu) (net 10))
 (segment (start 150.125 119.85) (end 151.175 119.85) (width 0.762) (layer F.Cu) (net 10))
 (segment (start 149.05 122.45) (end 149.05 120.925) (width 0.762) (layer F.Cu) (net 10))
 (segment (start 149.05 120.925) (end 150.125 119.85) (width 0.762) (layer F.Cu) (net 10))
 (segment (start 135.475 105.47) (end 135.475 107.145) (width 0.762) (layer F.Cu) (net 24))
 (segment (start 129.4875 99.15) (end 129.9625 99.15) (width 0.4064) (layer F.Cu) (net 2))
 (segment (start 129.4875 99.15) (end 129.984786 99.15) (width 0.25) (layer F.Cu) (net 2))
 (segment (start 130.5689 99.15) (end 132.0489 97.67) (width 0.4064) (layer F.Cu) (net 2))
 (segment (start 129.4875 99.15) (end 130.5689 99.15) (width 0.4064) (layer F.Cu) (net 2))
 (segment (start 136.4138 97.665) (end 136.4188 97.67) (width 0.762) (layer F.Cu) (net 2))
 (segment (start 132.385 97.665) (end 136.4138 97.665) (width 0.762) (layer F.Cu) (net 2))
 (segment (start 136.4188 97.67) (end 139.162 97.67) (width 0.762) (layer F.Cu) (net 2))
 (segment (start 155.6564 111.02) (end 157.025 112.3886) (width 0.4064) (layer F.Cu) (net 11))
 (segment (start 154.525 111.02) (end 155.6564 111.02) (width 0.4064) (layer F.Cu) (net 11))
 (segment (start 144.875 127.2) (end 151.175 127.2) (width 0.762) (layer F.Cu) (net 11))
 (segment (start 149.05 126.125) (end 149.05 124.6) (width 0.762) (layer F.Cu) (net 11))
 (segment (start 151.175 127.2) (end 150.125 127.2) (width 0.762) (layer F.Cu) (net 11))
 (segment (start 150.125 127.2) (end 149.05 126.125) (width 0.762) (layer F.Cu) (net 11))
 (segment (start 152 124.575) (end 149.075 124.575) (width 0.762) (layer F.Cu) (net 11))
 (segment (start 157.125 119.45) (end 152 124.575) (width 0.762) (layer F.Cu) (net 11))
 (segment (start 157.025 112.3886) (end 157.125 112.4886) (width 0.762) (layer F.Cu) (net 11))
 (segment (start 157.125 112.4886) (end 157.125 119.45) (width 0.762) (layer F.Cu) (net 11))
 (via (at 150.575 111.25) (size 0.8) (drill 0.4) (layers F.Cu B.Cu) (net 6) (status 40000))
 (segment (start 149.505 112.32) (end 148.625 112.32) (width 0.4064) (layer F.Cu) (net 6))
 (segment (start 150.575 111.25) (end 149.505 112.32) (width 0.4064) (layer F.Cu) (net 6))
 (segment (start 150.575 110.9) (end 149.55 109.875) (width 0.25) (layer B.Cu) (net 6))
 (segment (start 150.575 111.25) (end 150.575 110.9) (width 0.25) (layer B.Cu) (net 6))
 (segment (start 148.625 112.97) (end 148.1 112.97) (width 0.4064) (layer F.Cu) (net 7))
 (via (at 150.575 112.525) (size 0.8) (drill 0.4) (layers F.Cu B.Cu) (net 7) (status 40000))
 (segment (start 149.955 112.97) (end 150.4 112.525) (width 0.4064) (layer F.Cu) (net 7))
 (segment (start 148.625 112.97) (end 149.955 112.97) (width 0.4064) (layer F.Cu) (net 7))
 (segment (start 150.575 112.9) (end 149.55 113.925) (width 0.25) (layer B.Cu) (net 7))
 (segment (start 150.575 112.525) (end 150.575 112.9) (width 0.25) (layer B.Cu) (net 7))
 (via (at 152.575 112.525) (size 0.8) (drill 0.4) (layers F.Cu B.Cu) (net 9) (status 40000))
 (segment (start 152.78 112.32) (end 152.575 112.525) (width 0.4064) (layer F.Cu) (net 9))
 (segment (start 154.525 112.32) (end 152.78 112.32) (width 0.4064) (layer F.Cu) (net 9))
 (segment (start 152.575 112.9) (end 153.6 113.925) (width 0.25) (layer B.Cu) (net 9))
 (segment (start 152.575 112.525) (end 152.575 112.9) (width 0.25) (layer B.Cu) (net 9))
 (via (at 152.575 111.25) (size 0.8) (drill 0.4) (layers F.Cu B.Cu) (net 8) (status 40000))
 (segment (start 152.995 111.67) (end 152.575 111.25) (width 0.4064) (layer F.Cu) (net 8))
 (segment (start 154.525 111.67) (end 152.995 111.67) (width 0.4064) (layer F.Cu) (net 8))
 (segment (start 152.575 110.9) (end 153.6 109.875) (width 0.25) (layer B.Cu) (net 8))
 (segment (start 152.575 111.25) (end 152.575 110.9) (width 0.25) (layer B.Cu) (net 8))
 (segment (start 133.632 103.558) (end 135.229 103.558) (width 0.762) (layer F.Cu) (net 22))
 (segment (start 133.632 103.033) (end 133.632 103.558) (width 0.762) (layer F.Cu) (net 22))
 (segment (start 135.015 99.17) (end 135.015 101.65) (width 0.762) (layer F.Cu) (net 22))
 (segment (start 135.015 101.65) (end 133.632 103.033) (width 0.762) (layer F.Cu) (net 22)))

